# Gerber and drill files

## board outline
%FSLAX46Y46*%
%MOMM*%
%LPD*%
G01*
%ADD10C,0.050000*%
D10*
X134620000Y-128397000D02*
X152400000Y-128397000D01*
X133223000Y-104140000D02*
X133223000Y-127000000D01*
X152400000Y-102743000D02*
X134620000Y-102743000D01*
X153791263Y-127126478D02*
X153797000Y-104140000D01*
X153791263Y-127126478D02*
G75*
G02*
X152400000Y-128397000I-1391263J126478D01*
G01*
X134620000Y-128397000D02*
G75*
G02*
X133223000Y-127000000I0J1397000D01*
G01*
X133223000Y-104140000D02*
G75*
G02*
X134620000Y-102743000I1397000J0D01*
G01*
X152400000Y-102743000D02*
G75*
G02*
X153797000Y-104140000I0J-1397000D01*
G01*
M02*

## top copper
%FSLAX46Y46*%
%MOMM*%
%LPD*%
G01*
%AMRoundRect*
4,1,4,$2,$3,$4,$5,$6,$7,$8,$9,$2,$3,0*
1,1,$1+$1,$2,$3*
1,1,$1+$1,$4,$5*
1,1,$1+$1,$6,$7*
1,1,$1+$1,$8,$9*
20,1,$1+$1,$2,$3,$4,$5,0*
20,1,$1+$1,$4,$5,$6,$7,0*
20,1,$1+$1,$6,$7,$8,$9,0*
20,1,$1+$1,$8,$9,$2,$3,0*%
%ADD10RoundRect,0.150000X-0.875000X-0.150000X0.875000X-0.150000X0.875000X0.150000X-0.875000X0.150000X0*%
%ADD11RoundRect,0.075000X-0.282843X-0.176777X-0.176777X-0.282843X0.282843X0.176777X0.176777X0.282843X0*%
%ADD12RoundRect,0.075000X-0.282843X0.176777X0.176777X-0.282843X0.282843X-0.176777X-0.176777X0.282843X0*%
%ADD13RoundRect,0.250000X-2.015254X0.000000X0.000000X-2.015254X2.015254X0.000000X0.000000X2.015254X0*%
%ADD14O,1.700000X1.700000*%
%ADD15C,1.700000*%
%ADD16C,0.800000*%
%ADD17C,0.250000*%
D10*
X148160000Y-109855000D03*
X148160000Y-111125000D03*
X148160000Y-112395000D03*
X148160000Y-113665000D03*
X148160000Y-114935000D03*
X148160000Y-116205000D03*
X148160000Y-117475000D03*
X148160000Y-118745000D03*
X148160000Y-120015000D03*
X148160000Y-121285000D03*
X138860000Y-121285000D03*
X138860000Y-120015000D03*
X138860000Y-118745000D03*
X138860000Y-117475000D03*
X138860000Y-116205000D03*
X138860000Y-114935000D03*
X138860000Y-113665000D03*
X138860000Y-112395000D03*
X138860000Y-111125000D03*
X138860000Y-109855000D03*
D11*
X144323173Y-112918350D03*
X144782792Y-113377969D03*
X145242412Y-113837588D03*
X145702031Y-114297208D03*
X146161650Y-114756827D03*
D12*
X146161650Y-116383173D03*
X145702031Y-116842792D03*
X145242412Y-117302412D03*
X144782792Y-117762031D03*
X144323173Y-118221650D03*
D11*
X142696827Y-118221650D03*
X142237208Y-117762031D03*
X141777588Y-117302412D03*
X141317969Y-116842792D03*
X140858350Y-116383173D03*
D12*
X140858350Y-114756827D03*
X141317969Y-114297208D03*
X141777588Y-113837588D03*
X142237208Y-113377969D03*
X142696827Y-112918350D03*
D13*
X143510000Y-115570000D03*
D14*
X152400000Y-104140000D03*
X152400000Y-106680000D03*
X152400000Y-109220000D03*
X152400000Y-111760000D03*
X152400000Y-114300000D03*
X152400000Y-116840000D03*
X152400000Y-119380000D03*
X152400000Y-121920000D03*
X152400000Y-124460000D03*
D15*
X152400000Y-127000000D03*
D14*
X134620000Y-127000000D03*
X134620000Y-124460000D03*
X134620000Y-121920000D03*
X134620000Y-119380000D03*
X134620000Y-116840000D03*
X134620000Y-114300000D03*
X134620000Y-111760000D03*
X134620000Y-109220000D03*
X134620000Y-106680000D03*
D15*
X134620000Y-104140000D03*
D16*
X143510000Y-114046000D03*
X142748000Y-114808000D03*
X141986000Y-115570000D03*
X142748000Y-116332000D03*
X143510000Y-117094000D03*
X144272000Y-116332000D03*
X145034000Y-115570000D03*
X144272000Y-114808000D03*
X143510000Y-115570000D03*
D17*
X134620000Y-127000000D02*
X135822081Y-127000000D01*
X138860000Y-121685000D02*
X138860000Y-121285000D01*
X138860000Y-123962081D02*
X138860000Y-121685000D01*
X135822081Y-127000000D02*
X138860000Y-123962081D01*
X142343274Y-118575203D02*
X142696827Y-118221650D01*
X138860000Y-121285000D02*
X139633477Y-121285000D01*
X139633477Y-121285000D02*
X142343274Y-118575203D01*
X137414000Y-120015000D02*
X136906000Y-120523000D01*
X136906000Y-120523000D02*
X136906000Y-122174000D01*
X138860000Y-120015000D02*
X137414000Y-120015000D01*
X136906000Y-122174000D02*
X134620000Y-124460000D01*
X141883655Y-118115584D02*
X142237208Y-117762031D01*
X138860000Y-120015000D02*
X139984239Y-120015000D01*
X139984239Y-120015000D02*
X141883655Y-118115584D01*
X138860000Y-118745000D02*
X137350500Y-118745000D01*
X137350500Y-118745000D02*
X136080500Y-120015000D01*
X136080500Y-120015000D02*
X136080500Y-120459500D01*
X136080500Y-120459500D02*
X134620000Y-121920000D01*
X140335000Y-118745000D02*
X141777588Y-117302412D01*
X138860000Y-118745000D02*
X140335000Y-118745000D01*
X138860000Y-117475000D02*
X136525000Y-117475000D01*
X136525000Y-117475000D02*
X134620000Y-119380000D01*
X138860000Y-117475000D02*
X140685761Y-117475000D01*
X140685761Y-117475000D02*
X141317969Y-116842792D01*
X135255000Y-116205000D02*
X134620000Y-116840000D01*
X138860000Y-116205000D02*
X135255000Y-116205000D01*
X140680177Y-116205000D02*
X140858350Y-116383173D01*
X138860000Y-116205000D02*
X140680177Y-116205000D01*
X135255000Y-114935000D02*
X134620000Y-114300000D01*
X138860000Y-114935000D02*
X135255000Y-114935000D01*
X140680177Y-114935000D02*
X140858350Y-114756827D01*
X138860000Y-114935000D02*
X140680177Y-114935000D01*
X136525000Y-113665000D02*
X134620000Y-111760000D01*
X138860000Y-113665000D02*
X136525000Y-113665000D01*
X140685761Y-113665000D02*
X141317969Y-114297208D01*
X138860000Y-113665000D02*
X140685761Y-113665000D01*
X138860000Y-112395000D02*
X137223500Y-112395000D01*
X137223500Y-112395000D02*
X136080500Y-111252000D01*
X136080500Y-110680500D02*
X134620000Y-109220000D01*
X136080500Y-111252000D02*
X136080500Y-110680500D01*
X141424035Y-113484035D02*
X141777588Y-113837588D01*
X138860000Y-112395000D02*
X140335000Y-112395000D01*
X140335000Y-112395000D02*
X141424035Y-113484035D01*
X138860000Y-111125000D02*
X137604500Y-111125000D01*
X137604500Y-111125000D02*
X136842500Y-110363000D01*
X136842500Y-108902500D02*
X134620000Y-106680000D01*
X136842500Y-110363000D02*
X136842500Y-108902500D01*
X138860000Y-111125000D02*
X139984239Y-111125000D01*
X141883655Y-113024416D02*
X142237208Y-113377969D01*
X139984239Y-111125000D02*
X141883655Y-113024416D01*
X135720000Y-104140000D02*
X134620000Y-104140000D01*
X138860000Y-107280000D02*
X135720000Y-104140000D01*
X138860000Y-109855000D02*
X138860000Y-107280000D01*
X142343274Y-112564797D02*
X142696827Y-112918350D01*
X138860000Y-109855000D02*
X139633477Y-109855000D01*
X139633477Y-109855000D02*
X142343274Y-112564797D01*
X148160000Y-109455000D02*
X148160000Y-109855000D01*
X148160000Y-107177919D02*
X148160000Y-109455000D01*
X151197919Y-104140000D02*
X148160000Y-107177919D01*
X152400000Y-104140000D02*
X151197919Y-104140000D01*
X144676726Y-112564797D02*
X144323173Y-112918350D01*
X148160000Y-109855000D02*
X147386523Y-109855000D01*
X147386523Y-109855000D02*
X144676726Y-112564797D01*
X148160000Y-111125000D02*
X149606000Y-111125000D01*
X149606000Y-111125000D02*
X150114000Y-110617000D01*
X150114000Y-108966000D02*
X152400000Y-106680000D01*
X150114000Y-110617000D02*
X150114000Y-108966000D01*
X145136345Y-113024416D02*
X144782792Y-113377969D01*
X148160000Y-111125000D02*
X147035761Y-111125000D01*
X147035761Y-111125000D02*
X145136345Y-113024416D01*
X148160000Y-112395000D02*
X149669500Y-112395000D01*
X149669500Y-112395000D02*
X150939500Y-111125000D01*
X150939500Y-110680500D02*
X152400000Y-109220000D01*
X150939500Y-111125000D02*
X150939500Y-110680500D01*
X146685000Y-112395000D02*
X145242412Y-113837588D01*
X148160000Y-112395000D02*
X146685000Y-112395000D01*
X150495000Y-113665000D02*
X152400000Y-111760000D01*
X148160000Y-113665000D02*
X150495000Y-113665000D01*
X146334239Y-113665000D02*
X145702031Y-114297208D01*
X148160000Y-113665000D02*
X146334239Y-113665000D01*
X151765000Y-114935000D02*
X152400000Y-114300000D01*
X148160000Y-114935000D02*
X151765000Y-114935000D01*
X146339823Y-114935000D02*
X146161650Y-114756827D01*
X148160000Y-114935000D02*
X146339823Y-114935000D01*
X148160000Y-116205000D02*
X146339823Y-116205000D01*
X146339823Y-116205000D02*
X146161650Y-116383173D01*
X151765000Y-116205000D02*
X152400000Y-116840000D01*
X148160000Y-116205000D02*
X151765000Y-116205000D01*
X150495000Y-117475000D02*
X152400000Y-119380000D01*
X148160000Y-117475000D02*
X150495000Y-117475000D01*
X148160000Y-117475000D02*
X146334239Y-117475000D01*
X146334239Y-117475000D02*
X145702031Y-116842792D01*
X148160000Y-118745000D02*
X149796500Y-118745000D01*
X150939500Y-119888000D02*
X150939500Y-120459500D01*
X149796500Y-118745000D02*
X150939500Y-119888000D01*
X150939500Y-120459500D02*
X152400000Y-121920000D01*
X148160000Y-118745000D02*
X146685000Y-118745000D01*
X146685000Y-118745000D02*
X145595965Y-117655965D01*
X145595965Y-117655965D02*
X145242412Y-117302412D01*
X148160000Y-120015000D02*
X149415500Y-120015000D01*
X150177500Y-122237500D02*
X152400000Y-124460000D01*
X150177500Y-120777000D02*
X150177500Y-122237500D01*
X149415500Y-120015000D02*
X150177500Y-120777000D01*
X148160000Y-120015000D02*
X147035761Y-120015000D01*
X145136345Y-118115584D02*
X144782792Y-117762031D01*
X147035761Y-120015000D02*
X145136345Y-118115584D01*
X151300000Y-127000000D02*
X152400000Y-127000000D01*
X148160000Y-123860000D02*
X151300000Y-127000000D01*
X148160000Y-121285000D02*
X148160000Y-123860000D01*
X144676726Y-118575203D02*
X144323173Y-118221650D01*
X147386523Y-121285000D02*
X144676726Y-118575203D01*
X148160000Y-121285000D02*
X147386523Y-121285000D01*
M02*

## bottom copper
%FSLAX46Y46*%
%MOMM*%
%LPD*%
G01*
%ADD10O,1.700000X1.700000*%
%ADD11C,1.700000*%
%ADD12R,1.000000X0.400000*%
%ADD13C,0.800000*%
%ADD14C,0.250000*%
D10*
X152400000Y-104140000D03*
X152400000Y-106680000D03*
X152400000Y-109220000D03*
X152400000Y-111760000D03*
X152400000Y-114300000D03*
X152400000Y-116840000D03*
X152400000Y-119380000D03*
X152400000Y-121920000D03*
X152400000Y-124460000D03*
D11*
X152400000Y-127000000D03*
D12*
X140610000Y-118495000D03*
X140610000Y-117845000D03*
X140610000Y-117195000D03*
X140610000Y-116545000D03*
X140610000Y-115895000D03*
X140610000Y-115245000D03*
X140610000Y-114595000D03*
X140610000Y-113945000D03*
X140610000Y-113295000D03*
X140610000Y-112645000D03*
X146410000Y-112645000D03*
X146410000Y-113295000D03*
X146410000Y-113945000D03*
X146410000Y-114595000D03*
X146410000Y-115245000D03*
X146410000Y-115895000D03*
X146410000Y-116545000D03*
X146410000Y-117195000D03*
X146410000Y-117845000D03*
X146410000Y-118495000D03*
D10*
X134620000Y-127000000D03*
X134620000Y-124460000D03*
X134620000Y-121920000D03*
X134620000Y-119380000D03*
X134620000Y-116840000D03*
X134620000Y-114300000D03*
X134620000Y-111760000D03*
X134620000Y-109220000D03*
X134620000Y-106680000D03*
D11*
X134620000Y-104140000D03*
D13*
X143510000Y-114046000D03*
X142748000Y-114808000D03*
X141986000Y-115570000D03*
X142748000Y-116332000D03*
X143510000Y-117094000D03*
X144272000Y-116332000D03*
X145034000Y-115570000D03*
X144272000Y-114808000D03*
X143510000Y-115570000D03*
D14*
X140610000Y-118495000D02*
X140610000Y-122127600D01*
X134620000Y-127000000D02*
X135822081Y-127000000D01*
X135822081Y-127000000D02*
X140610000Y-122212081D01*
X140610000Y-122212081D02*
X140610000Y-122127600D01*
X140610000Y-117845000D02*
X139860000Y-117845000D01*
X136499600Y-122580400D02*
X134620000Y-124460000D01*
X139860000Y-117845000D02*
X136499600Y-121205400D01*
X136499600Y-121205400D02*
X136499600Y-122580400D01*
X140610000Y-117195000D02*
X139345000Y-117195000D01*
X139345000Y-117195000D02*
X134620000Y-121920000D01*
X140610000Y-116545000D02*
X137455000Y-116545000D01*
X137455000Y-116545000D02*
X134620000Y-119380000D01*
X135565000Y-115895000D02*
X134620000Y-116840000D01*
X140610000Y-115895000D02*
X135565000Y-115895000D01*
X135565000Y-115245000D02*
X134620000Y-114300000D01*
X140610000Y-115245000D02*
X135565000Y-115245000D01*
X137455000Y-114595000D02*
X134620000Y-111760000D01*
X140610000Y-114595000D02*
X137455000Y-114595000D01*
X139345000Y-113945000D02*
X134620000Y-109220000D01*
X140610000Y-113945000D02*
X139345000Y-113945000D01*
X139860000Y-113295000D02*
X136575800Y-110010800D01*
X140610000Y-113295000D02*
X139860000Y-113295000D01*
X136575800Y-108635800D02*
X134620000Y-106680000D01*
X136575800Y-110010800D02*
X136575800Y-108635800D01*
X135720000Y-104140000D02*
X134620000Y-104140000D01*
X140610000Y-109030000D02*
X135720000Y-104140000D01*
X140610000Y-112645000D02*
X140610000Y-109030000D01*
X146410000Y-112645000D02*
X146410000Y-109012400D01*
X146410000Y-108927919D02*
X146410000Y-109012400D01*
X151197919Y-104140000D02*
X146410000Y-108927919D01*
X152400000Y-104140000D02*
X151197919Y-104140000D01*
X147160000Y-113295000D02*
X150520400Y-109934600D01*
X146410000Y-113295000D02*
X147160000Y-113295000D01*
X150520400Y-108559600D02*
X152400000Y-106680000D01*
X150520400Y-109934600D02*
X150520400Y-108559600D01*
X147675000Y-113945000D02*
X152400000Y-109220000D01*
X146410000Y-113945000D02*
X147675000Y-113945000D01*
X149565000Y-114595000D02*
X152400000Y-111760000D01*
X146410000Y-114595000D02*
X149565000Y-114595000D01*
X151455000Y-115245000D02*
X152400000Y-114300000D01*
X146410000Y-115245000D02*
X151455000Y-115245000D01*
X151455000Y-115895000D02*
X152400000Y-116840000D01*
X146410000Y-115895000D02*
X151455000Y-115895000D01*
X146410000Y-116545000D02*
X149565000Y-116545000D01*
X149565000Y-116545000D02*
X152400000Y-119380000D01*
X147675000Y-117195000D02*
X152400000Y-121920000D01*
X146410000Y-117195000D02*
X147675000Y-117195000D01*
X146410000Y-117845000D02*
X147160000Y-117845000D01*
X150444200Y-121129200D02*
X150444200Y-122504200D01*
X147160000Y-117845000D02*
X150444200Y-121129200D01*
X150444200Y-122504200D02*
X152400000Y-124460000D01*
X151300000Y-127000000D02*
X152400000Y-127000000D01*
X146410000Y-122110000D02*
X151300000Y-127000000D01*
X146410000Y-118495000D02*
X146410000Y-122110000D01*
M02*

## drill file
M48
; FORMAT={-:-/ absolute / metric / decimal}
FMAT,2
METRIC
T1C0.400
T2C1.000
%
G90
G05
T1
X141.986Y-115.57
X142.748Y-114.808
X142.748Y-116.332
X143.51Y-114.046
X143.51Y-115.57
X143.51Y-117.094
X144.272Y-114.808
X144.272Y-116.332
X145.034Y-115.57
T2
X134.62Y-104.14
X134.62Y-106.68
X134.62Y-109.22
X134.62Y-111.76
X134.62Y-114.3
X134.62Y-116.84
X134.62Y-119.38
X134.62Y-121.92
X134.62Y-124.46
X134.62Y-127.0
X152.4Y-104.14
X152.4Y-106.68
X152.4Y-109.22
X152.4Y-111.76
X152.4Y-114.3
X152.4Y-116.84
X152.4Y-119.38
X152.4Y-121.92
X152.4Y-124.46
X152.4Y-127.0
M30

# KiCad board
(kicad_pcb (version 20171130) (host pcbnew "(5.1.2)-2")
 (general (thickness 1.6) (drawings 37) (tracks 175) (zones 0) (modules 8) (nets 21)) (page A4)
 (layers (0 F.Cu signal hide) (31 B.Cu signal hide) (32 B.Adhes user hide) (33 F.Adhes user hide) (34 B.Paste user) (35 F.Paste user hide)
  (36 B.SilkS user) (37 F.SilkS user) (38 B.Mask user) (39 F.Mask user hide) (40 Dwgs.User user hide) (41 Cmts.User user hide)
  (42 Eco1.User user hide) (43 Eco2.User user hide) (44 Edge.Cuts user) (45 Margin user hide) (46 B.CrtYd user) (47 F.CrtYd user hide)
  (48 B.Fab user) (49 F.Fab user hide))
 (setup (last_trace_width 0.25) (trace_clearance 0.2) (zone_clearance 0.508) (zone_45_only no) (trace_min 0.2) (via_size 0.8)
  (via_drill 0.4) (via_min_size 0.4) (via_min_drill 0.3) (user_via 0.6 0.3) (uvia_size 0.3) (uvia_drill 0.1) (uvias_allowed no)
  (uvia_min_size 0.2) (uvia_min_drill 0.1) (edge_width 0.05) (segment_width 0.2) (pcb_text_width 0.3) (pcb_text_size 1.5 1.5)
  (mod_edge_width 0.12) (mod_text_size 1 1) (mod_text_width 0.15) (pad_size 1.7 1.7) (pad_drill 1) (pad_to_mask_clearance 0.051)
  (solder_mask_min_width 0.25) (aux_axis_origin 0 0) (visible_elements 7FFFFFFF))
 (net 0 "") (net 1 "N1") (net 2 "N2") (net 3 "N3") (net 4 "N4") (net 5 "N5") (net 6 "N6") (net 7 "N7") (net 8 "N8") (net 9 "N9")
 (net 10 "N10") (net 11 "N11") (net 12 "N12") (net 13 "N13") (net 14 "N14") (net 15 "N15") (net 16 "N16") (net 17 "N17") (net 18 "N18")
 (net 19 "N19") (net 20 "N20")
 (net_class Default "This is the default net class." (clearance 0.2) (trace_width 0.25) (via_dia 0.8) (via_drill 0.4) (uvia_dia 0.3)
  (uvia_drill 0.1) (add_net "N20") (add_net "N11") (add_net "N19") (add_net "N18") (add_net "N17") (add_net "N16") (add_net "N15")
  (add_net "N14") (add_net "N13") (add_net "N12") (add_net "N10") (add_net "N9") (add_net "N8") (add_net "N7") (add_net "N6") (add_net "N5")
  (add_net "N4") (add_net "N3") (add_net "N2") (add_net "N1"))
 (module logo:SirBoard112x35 (layer B.Cu) (at 143.51 108.331)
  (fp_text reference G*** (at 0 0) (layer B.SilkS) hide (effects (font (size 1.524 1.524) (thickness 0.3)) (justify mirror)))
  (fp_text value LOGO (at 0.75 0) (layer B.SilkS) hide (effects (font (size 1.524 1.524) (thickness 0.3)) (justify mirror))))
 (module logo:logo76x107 (layer B.Cu) (at 143.51 123.952)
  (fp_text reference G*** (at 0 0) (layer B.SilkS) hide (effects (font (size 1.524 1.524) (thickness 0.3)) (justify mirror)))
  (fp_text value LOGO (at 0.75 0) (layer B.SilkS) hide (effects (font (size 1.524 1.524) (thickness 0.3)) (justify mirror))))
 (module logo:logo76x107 (layer F.Cu) (at 143.51 106.172 90)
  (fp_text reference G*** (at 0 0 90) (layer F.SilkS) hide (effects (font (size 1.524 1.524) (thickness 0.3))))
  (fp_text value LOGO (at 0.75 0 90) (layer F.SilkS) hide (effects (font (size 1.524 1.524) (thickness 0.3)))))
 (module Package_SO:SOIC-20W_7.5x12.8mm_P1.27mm (layer F.Cu) (at 143.51 115.57)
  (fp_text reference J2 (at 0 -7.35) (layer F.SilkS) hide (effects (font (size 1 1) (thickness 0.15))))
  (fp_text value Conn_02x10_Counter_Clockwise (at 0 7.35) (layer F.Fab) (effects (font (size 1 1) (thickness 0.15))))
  (pad 20 smd roundrect (at 4.65 -5.715) (size 2.05 0.6) (layers F.Cu F.Paste F.Mask) (roundrect_rratio 0.25) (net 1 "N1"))
  (pad 19 smd roundrect (at 4.65 -4.445) (size 2.05 0.6) (layers F.Cu F.Paste F.Mask) (roundrect_rratio 0.25) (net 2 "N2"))
  (pad 18 smd roundrect (at 4.65 -3.175) (size 2.05 0.6) (layers F.Cu F.Paste F.Mask) (roundrect_rratio 0.25) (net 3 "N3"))
  (pad 17 smd roundrect (at 4.65 -1.905) (size 2.05 0.6) (layers F.Cu F.Paste F.Mask) (roundrect_rratio 0.25) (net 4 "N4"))
  (pad 16 smd roundrect (at 4.65 -0.635) (size 2.05 0.6) (layers F.Cu F.Paste F.Mask) (roundrect_rratio 0.25) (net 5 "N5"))
  (pad 15 smd roundrect (at 4.65 0.635) (size 2.05 0.6) (layers F.Cu F.Paste F.Mask) (roundrect_rratio 0.25) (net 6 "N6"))
  (pad 14 smd roundrect (at 4.65 1.905) (size 2.05 0.6) (layers F.Cu F.Paste F.Mask) (roundrect_rratio 0.25) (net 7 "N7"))
  (pad 13 smd roundrect (at 4.65 3.175) (size 2.05 0.6) (layers F.Cu F.Paste F.Mask) (roundrect_rratio 0.25) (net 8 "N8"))
  (pad 12 smd roundrect (at 4.65 4.445) (size 2.05 0.6) (layers F.Cu F.Paste F.Mask) (roundrect_rratio 0.25) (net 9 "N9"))
  (pad 11 smd roundrect (at 4.65 5.715) (size 2.05 0.6) (layers F.Cu F.Paste F.Mask) (roundrect_rratio 0.25) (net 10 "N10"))
  (pad 10 smd roundrect (at -4.65 5.715) (size 2.05 0.6) (layers F.Cu F.Paste F.Mask) (roundrect_rratio 0.25) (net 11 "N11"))
  (pad 9 smd roundrect (at -4.65 4.445) (size 2.05 0.6) (layers F.Cu F.Paste F.Mask) (roundrect_rratio 0.25) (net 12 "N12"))
  (pad 8 smd roundrect (at -4.65 3.175) (size 2.05 0.6) (layers F.Cu F.Paste F.Mask) (roundrect_rratio 0.25) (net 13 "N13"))
  (pad 7 smd roundrect (at -4.65 1.905) (size 2.05 0.6) (layers F.Cu F.Paste F.Mask) (roundrect_rratio 0.25) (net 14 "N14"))
  (pad 6 smd roundrect (at -4.65 0.635) (size 2.05 0.6) (layers F.Cu F.Paste F.Mask) (roundrect_rratio 0.25) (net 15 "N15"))
  (pad 5 smd roundrect (at -4.65 -0.635) (size 2.05 0.6) (layers F.Cu F.Paste F.Mask) (roundrect_rratio 0.25) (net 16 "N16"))
  (pad 4 smd roundrect (at -4.65 -1.905) (size 2.05 0.6) (layers F.Cu F.Paste F.Mask) (roundrect_rratio 0.25) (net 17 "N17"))
  (pad 3 smd roundrect (at -4.65 -3.175) (size 2.05 0.6) (layers F.Cu F.Paste F.Mask) (roundrect_rratio 0.25) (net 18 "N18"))
  (pad 2 smd roundrect (at -4.65 -4.445) (size 2.05 0.6) (layers F.Cu F.Paste F.Mask) (roundrect_rratio 0.25) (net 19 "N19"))
  (pad 1 smd roundrect (at -4.65 -5.715) (size 2.05 0.6) (layers F.Cu F.Paste F.Mask) (roundrect_rratio 0.25) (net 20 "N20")))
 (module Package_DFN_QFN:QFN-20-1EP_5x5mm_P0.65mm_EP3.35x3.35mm (layer F.Cu) (at 143.51 115.57 315)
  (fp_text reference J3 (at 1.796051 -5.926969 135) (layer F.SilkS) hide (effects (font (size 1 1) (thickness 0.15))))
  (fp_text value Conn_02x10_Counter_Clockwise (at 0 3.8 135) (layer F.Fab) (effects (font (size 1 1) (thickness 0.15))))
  (pad 20 smd roundrect (at -1.3 -2.45 315) (size 0.3 0.8) (layers F.Cu F.Paste F.Mask) (roundrect_rratio 0.25) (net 1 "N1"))
  (pad 19 smd roundrect (at -0.65 -2.45 315) (size 0.3 0.8) (layers F.Cu F.Paste F.Mask) (roundrect_rratio 0.25) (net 2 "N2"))
  (pad 18 smd roundrect (at 0 -2.45 315) (size 0.3 0.8) (layers F.Cu F.Paste F.Mask) (roundrect_rratio 0.25) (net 3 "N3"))
  (pad 17 smd roundrect (at 0.65 -2.45 315) (size 0.3 0.8) (layers F.Cu F.Paste F.Mask) (roundrect_rratio 0.25) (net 4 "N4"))
  (pad 16 smd roundrect (at 1.3 -2.45 315) (size 0.3 0.8) (layers F.Cu F.Paste F.Mask) (roundrect_rratio 0.25) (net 5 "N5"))
  (pad 15 smd roundrect (at 2.45 -1.3 315) (size 0.8 0.3) (layers F.Cu F.Paste F.Mask) (roundrect_rratio 0.25) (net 6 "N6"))
  (pad 14 smd roundrect (at 2.45 -0.65 315) (size 0.8 0.3) (layers F.Cu F.Paste F.Mask) (roundrect_rratio 0.25) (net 7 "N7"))
  (pad 13 smd roundrect (at 2.45 0 315) (size 0.8 0.3) (layers F.Cu F.Paste F.Mask) (roundrect_rratio 0.25) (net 8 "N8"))
  (pad 12 smd roundrect (at 2.45 0.65 315) (size 0.8 0.3) (layers F.Cu F.Paste F.Mask) (roundrect_rratio 0.25) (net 9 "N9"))
  (pad 11 smd roundrect (at 2.45 1.3 315) (size 0.8 0.3) (layers F.Cu F.Paste F.Mask) (roundrect_rratio 0.25) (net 10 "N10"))
  (pad 10 smd roundrect (at 1.3 2.45 315) (size 0.3 0.8) (layers F.Cu F.Paste F.Mask) (roundrect_rratio 0.25) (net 11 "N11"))
  (pad 9 smd roundrect (at 0.65 2.45 315) (size 0.3 0.8) (layers F.Cu F.Paste F.Mask) (roundrect_rratio 0.25) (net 12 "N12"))
  (pad 8 smd roundrect (at 0 2.45 315) (size 0.3 0.8) (layers F.Cu F.Paste F.Mask) (roundrect_rratio 0.25) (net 13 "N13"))
  (pad 7 smd roundrect (at -0.65 2.45 315) (size 0.3 0.8) (layers F.Cu F.Paste F.Mask) (roundrect_rratio 0.25) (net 14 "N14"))
  (pad 6 smd roundrect (at -1.3 2.45 315) (size 0.3 0.8) (layers F.Cu F.Paste F.Mask) (roundrect_rratio 0.25) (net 15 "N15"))
  (pad 5 smd roundrect (at -2.45 1.3 315) (size 0.8 0.3) (layers F.Cu F.Paste F.Mask) (roundrect_rratio 0.25) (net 16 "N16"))
  (pad 4 smd roundrect (at -2.45 0.65 315) (size 0.8 0.3) (layers F.Cu F.Paste F.Mask) (roundrect_rratio 0.25) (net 17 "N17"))
  (pad 3 smd roundrect (at -2.45 0 315) (size 0.8 0.3) (layers F.Cu F.Paste F.Mask) (roundrect_rratio 0.25) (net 18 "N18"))
  (pad 2 smd roundrect (at -2.45 -0.65 315) (size 0.8 0.3) (layers F.Cu F.Paste F.Mask) (roundrect_rratio 0.25) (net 19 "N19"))
  (pad 1 smd roundrect (at -2.45 -1.3 315) (size 0.8 0.3) (layers F.Cu F.Paste F.Mask) (roundrect_rratio 0.25) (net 20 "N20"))
  (pad "" smd roundrect (at 0.84 0.84 315) (size 1.35 1.35) (layers F.Paste) (roundrect_rratio 0.185185))
  (pad "" smd roundrect (at 0.84 -0.84 315) (size 1.35 1.35) (layers F.Paste) (roundrect_rratio 0.185185))
  (pad "" smd roundrect (at -0.84 0.84 315) (size 1.35 1.35) (layers F.Paste) (roundrect_rratio 0.185185))
  (pad "" smd roundrect (at -0.84 -0.84 315) (size 1.35 1.35) (layers F.Paste) (roundrect_rratio 0.185185))
  (pad 21 smd roundrect (at 0 0 315) (size 3.35 3.35) (layers F.Cu F.Mask) (roundrect_rratio 0.074627)))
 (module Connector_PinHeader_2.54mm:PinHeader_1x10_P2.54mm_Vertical (layer F.Cu) (at 152.4 127 180)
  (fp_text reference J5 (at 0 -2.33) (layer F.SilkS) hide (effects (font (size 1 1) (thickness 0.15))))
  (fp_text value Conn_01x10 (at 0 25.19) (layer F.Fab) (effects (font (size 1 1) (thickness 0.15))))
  (pad 10 thru_hole oval (at 0 22.86 180) (size 1.7 1.7) (drill 1) (layers *.Cu *.Mask) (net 1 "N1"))
  (pad 9 thru_hole oval (at 0 20.32 180) (size 1.7 1.7) (drill 1) (layers *.Cu *.Mask) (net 2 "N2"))
  (pad 8 thru_hole oval (at 0 17.78 180) (size 1.7 1.7) (drill 1) (layers *.Cu *.Mask) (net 3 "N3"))
  (pad 7 thru_hole oval (at 0 15.24 180) (size 1.7 1.7) (drill 1) (layers *.Cu *.Mask) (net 4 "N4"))
  (pad 6 thru_hole oval (at 0 12.7 180) (size 1.7 1.7) (drill 1) (layers *.Cu *.Mask) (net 5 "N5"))
  (pad 5 thru_hole oval (at 0 10.16 180) (size 1.7 1.7) (drill 1) (layers *.Cu *.Mask) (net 6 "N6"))
  (pad 4 thru_hole oval (at 0 7.62 180) (size 1.7 1.7) (drill 1) (layers *.Cu *.Mask) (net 7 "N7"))
  (pad 3 thru_hole oval (at 0 5.08 180) (size 1.7 1.7) (drill 1) (layers *.Cu *.Mask) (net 8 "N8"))
  (pad 2 thru_hole oval (at 0 2.54 180) (size 1.7 1.7) (drill 1) (layers *.Cu *.Mask) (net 9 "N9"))
  (pad 1 thru_hole circle (at 0 0 180) (size 1.7 1.7) (drill 1) (layers *.Cu *.Mask) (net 10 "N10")))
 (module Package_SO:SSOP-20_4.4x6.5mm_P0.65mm (layer B.Cu) (at 143.51 115.57)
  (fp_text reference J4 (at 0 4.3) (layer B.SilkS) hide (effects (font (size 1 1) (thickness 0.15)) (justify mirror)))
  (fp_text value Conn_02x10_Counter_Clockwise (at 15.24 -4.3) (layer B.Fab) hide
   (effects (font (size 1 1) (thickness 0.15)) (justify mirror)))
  (pad 1 smd rect (at -2.9 2.925) (size 1 0.4) (layers B.Cu B.Paste B.Mask) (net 11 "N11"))
  (pad 2 smd rect (at -2.9 2.275) (size 1 0.4) (layers B.Cu B.Paste B.Mask) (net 12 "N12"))
  (pad 3 smd rect (at -2.9 1.625) (size 1 0.4) (layers B.Cu B.Paste B.Mask) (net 13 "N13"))
  (pad 4 smd rect (at -2.9 0.975) (size 1 0.4) (layers B.Cu B.Paste B.Mask) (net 14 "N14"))
  (pad 5 smd rect (at -2.9 0.325) (size 1 0.4) (layers B.Cu B.Paste B.Mask) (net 15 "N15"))
  (pad 6 smd rect (at -2.9 -0.325) (size 1 0.4) (layers B.Cu B.Paste B.Mask) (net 16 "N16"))
  (pad 7 smd rect (at -2.9 -0.975) (size 1 0.4) (layers B.Cu B.Paste B.Mask) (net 17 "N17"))
  (pad 8 smd rect (at -2.9 -1.625) (size 1 0.4) (layers B.Cu B.Paste B.Mask) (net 18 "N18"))
  (pad 9 smd rect (at -2.9 -2.275) (size 1 0.4) (layers B.Cu B.Paste B.Mask) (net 19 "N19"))
  (pad 10 smd rect (at -2.9 -2.925) (size 1 0.4) (layers B.Cu B.Paste B.Mask) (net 20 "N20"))
  (pad 11 smd rect (at 2.9 -2.925) (size 1 0.4) (layers B.Cu B.Paste B.Mask) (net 1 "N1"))
  (pad 12 smd rect (at 2.9 -2.275) (size 1 0.4) (layers B.Cu B.Paste B.Mask) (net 2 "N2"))
  (pad 13 smd rect (at 2.9 -1.625) (size 1 0.4) (layers B.Cu B.Paste B.Mask) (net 3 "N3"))
  (pad 14 smd rect (at 2.9 -0.975) (size 1 0.4) (layers B.Cu B.Paste B.Mask) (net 4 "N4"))
  (pad 15 smd rect (at 2.9 -0.325) (size 1 0.4) (layers B.Cu B.Paste B.Mask) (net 5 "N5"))
  (pad 16 smd rect (at 2.9 0.325) (size 1 0.4) (layers B.Cu B.Paste B.Mask) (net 6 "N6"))
  (pad 17 smd rect (at 2.9 0.975) (size 1 0.4) (layers B.Cu B.Paste B.Mask) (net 7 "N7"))
  (pad 18 smd rect (at 2.9 1.625) (size 1 0.4) (layers B.Cu B.Paste B.Mask) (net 8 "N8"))
  (pad 19 smd rect (at 2.9 2.275) (size 1 0.4) (layers B.Cu B.Paste B.Mask) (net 9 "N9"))
  (pad 20 smd rect (at 2.9 2.925) (size 1 0.4) (layers B.Cu B.Paste B.Mask) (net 10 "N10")))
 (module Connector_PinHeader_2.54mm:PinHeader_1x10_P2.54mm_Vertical (layer F.Cu) (at 134.62 104.14)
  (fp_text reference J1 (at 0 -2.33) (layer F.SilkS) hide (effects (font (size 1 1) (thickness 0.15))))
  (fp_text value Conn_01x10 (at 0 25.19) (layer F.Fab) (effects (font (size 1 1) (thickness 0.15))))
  (pad 10 thru_hole oval (at 0 22.86) (size 1.7 1.7) (drill 1) (layers *.Cu *.Mask) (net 11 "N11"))
  (pad 9 thru_hole oval (at 0 20.32) (size 1.7 1.7) (drill 1) (layers *.Cu *.Mask) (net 12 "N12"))
  (pad 8 thru_hole oval (at 0 17.78) (size 1.7 1.7) (drill 1) (layers *.Cu *.Mask) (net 13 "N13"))
  (pad 7 thru_hole oval (at 0 15.24) (size 1.7 1.7) (drill 1) (layers *.Cu *.Mask) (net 14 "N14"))
  (pad 6 thru_hole oval (at 0 12.7) (size 1.7 1.7) (drill 1) (layers *.Cu *.Mask) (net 15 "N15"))
  (pad 5 thru_hole oval (at 0 10.16) (size 1.7 1.7) (drill 1) (layers *.Cu *.Mask) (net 16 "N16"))
  (pad 4 thru_hole oval (at 0 7.62) (size 1.7 1.7) (drill 1) (layers *.Cu *.Mask) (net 17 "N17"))
  (pad 3 thru_hole oval (at 0 5.08) (size 1.7 1.7) (drill 1) (layers *.Cu *.Mask) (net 18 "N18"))
  (pad 2 thru_hole oval (at 0 2.54) (size 1.7 1.7) (drill 1) (layers *.Cu *.Mask) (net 19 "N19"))
  (pad 1 thru_hole circle (at 0 0) (size 1.7 1.7) (drill 1) (layers *.Cu *.Mask) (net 20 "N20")))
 (gr_line (start 134.62 128.397) (end 152.4 128.397) (layer Edge.Cuts) (width 0.05))
 (gr_line (start 133.223 104.14) (end 133.223 127) (layer Edge.Cuts) (width 0.05))
 (gr_line (start 152.4 102.743) (end 134.62 102.743) (layer Edge.Cuts) (width 0.05))
 (gr_line (start 153.791263 127.126478) (end 153.797 104.14) (layer Edge.Cuts) (width 0.05))
 (gr_arc (start 152.4 127) (end 152.4 128.397) (angle -84.80557109) (layer Edge.Cuts) (width 0.05))
 (gr_arc (start 134.62 127) (end 133.223 127) (angle -90) (layer Edge.Cuts) (width 0.05))
 (gr_arc (start 134.62 104.14) (end 134.62 102.743) (angle -90) (layer Edge.Cuts) (width 0.05))
 (gr_arc (start 152.4 104.14) (end 153.797 104.14) (angle -90) (layer Edge.Cuts) (width 0.05))
 (via (at 143.51 114.046) (size 0.8) (drill 0.4) (layers F.Cu B.Cu) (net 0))
 (via (at 142.748 114.808) (size 0.8) (drill 0.4) (layers F.Cu B.Cu) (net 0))
 (via (at 141.986 115.57) (size 0.8) (drill 0.4) (layers F.Cu B.Cu) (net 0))
 (via (at 142.748 116.332) (size 0.8) (drill 0.4) (layers F.Cu B.Cu) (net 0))
 (via (at 143.51 117.094) (size 0.8) (drill 0.4) (layers F.Cu B.Cu) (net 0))
 (via (at 144.272 116.332) (size 0.8) (drill 0.4) (layers F.Cu B.Cu) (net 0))
 (via (at 145.034 115.57) (size 0.8) (drill 0.4) (layers F.Cu B.Cu) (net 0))
 (via (at 144.272 114.808) (size 0.8) (drill 0.4) (layers F.Cu B.Cu) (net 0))
 (via (at 143.51 115.57) (size 0.8) (drill 0.4) (layers F.Cu B.Cu) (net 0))
 (segment (start 134.62 127) (end 135.822081 127) (width 0.25) (layer F.Cu) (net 11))
 (segment (start 138.86 121.685) (end 138.86 121.285) (width 0.25) (layer F.Cu) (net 11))
 (segment (start 138.86 123.962081) (end 138.86 121.685) (width 0.25) (layer F.Cu) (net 11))
 (segment (start 135.822081 127) (end 138.86 123.962081) (width 0.25) (layer F.Cu) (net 11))
 (segment (start 142.343274 118.575203) (end 142.696827 118.22165) (width 0.25) (layer F.Cu) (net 11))
 (segment (start 138.86 121.285) (end 139.633477 121.285) (width 0.25) (layer F.Cu) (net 11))
 (segment (start 139.633477 121.285) (end 142.343274 118.575203) (width 0.25) (layer F.Cu) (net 11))
 (segment (start 140.61 118.495) (end 140.61 122.1276) (width 0.25) (layer B.Cu) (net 11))
 (segment (start 134.62 127) (end 135.822081 127) (width 0.25) (layer B.Cu) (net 11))
 (segment (start 135.822081 127) (end 140.61 122.212081) (width 0.25) (layer B.Cu) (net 11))
 (segment (start 140.61 122.212081) (end 140.61 122.1276) (width 0.25) (layer B.Cu) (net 11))
 (segment (start 137.414 120.015) (end 136.906 120.523) (width 0.25) (layer F.Cu) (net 12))
 (segment (start 136.906 120.523) (end 136.906 122.174) (width 0.25) (layer F.Cu) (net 12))
 (segment (start 138.86 120.015) (end 137.414 120.015) (width 0.25) (layer F.Cu) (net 12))
 (segment (start 136.906 122.174) (end 134.62 124.46) (width 0.25) (layer F.Cu) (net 12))
 (segment (start 141.883655 118.115584) (end 142.237208 117.762031) (width 0.25) (layer F.Cu) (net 12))
 (segment (start 138.86 120.015) (end 139.984239 120.015) (width 0.25) (layer F.Cu) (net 12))
 (segment (start 139.984239 120.015) (end 141.883655 118.115584) (width 0.25) (layer F.Cu) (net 12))
 (segment (start 140.61 117.845) (end 139.86 117.845) (width 0.25) (layer B.Cu) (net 12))
 (segment (start 136.4996 122.5804) (end 134.62 124.46) (width 0.25) (layer B.Cu) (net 12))
 (segment (start 139.86 117.845) (end 136.4996 121.2054) (width 0.25) (layer B.Cu) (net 12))
 (segment (start 136.4996 121.2054) (end 136.4996 122.5804) (width 0.25) (layer B.Cu) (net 12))
 (segment (start 138.86 118.745) (end 137.3505 118.745) (width 0.25) (layer F.Cu) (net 13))
 (segment (start 137.3505 118.745) (end 136.0805 120.015) (width 0.25) (layer F.Cu) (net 13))
 (segment (start 136.0805 120.015) (end 136.0805 120.4595) (width 0.25) (layer F.Cu) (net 13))
 (segment (start 136.0805 120.4595) (end 134.62 121.92) (width 0.25) (layer F.Cu) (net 13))
 (segment (start 140.335 118.745) (end 141.777588 117.302412) (width 0.25) (layer F.Cu) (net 13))
 (segment (start 138.86 118.745) (end 140.335 118.745) (width 0.25) (layer F.Cu) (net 13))
 (segment (start 140.61 117.195) (end 139.345 117.195) (width 0.25) (layer B.Cu) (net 13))
 (segment (start 139.345 117.195) (end 134.62 121.92) (width 0.25) (layer B.Cu) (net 13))
 (segment (start 138.86 117.475) (end 136.525 117.475) (width 0.25) (layer F.Cu) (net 14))
 (segment (start 136.525 117.475) (end 134.62 119.38) (width 0.25) (layer F.Cu) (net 14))
 (segment (start 138.86 117.475) (end 140.685761 117.475) (width 0.25) (layer F.Cu) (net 14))
 (segment (start 140.685761 117.475) (end 141.317969 116.842792) (width 0.25) (layer F.Cu) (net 14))
 (segment (start 140.61 116.545) (end 137.455 116.545) (width 0.25) (layer B.Cu) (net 14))
 (segment (start 137.455 116.545) (end 134.62 119.38) (width 0.25) (layer B.Cu) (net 14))
 (segment (start 135.255 116.205) (end 134.62 116.84) (width 0.25) (layer F.Cu) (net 15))
 (segment (start 138.86 116.205) (end 135.255 116.205) (width 0.25) (layer F.Cu) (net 15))
 (segment (start 140.680177 116.205) (end 140.85835 116.383173) (width 0.25) (layer F.Cu) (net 15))
 (segment (start 138.86 116.205) (end 140.680177 116.205) (width 0.25) (layer F.Cu) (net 15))
 (segment (start 135.565 115.895) (end 134.62 116.84) (width 0.25) (layer B.Cu) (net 15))
 (segment (start 140.61 115.895) (end 135.565 115.895) (width 0.25) (layer B.Cu) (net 15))
 (segment (start 135.255 114.935) (end 134.62 114.3) (width 0.25) (layer F.Cu) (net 16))
 (segment (start 138.86 114.935) (end 135.255 114.935) (width 0.25) (layer F.Cu) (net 16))
 (segment (start 140.680177 114.935) (end 140.85835 114.756827) (width 0.25) (layer F.Cu) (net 16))
 (segment (start 138.86 114.935) (end 140.680177 114.935) (width 0.25) (layer F.Cu) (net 16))
 (segment (start 135.565 115.245) (end 134.62 114.3) (width 0.25) (layer B.Cu) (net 16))
 (segment (start 140.61 115.245) (end 135.565 115.245) (width 0.25) (layer B.Cu) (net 16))
 (segment (start 136.525 113.665) (end 134.62 111.76) (width 0.25) (layer F.Cu) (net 17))
 (segment (start 138.86 113.665) (end 136.525 113.665) (width 0.25) (layer F.Cu) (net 17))
 (segment (start 140.685761 113.665) (end 141.317969 114.297208) (width 0.25) (layer F.Cu) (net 17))
 (segment (start 138.86 113.665) (end 140.685761 113.665) (width 0.25) (layer F.Cu) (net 17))
 (segment (start 137.455 114.595) (end 134.62 111.76) (width 0.25) (layer B.Cu) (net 17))
 (segment (start 140.61 114.595) (end 137.455 114.595) (width 0.25) (layer B.Cu) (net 17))
 (segment (start 138.86 112.395) (end 137.2235 112.395) (width 0.25) (layer F.Cu) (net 18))
 (segment (start 137.2235 112.395) (end 136.0805 111.252) (width 0.25) (layer F.Cu) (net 18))
 (segment (start 136.0805 110.6805) (end 134.62 109.22) (width 0.25) (layer F.Cu) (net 18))
 (segment (start 136.0805 111.252) (end 136.0805 110.6805) (width 0.25) (layer F.Cu) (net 18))
 (segment (start 141.424035 113.484035) (end 141.777588 113.837588) (width 0.25) (layer F.Cu) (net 18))
 (segment (start 138.86 112.395) (end 140.335 112.395) (width 0.25) (layer F.Cu) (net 18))
 (segment (start 140.335 112.395) (end 141.424035 113.484035) (width 0.25) (layer F.Cu) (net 18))
 (segment (start 139.345 113.945) (end 134.62 109.22) (width 0.25) (layer B.Cu) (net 18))
 (segment (start 140.61 113.945) (end 139.345 113.945) (width 0.25) (layer B.Cu) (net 18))
 (segment (start 138.86 111.125) (end 137.6045 111.125) (width 0.25) (layer F.Cu) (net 19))
 (segment (start 137.6045 111.125) (end 136.8425 110.363) (width 0.25) (layer F.Cu) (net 19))
 (segment (start 136.8425 108.9025) (end 134.62 106.68) (width 0.25) (layer F.Cu) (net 19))
 (segment (start 136.8425 110.363) (end 136.8425 108.9025) (width 0.25) (layer F.Cu) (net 19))
 (segment (start 138.86 111.125) (end 139.984239 111.125) (width 0.25) (layer F.Cu) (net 19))
 (segment (start 141.883655 113.024416) (end 142.237208 113.377969) (width 0.25) (layer F.Cu) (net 19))
 (segment (start 139.984239 111.125) (end 141.883655 113.024416) (width 0.25) (layer F.Cu) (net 19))
 (segment (start 139.86 113.295) (end 136.5758 110.0108) (width 0.25) (layer B.Cu) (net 19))
 (segment (start 140.61 113.295) (end 139.86 113.295) (width 0.25) (layer B.Cu) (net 19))
 (segment (start 136.5758 108.6358) (end 134.62 106.68) (width 0.25) (layer B.Cu) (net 19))
 (segment (start 136.5758 110.0108) (end 136.5758 108.6358) (width 0.25) (layer B.Cu) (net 19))
 (segment (start 135.72 104.14) (end 134.62 104.14) (width 0.25) (layer F.Cu) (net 20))
 (segment (start 138.86 107.28) (end 135.72 104.14) (width 0.25) (layer F.Cu) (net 20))
 (segment (start 138.86 109.855) (end 138.86 107.28) (width 0.25) (layer F.Cu) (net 20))
 (segment (start 142.343274 112.564797) (end 142.696827 112.91835) (width 0.25) (layer F.Cu) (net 20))
 (segment (start 138.86 109.855) (end 139.633477 109.855) (width 0.25) (layer F.Cu) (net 20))
 (segment (start 139.633477 109.855) (end 142.343274 112.564797) (width 0.25) (layer F.Cu) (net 20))
 (segment (start 135.72 104.14) (end 134.62 104.14) (width 0.25) (layer B.Cu) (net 20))
 (segment (start 140.61 109.03) (end 135.72 104.14) (width 0.25) (layer B.Cu) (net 20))
 (segment (start 140.61 112.645) (end 140.61 109.03) (width 0.25) (layer B.Cu) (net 20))
 (segment (start 148.16 109.455) (end 148.16 109.855) (width 0.25) (layer F.Cu) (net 1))
 (segment (start 148.16 107.177919) (end 148.16 109.455) (width 0.25) (layer F.Cu) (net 1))
 (segment (start 151.197919 104.14) (end 148.16 107.177919) (width 0.25) (layer F.Cu) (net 1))
 (segment (start 152.4 104.14) (end 151.197919 104.14) (width 0.25) (layer F.Cu) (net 1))
 (segment (start 144.676726 112.564797) (end 144.323173 112.91835) (width 0.25) (layer F.Cu) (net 1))
 (segment (start 148.16 109.855) (end 147.386523 109.855) (width 0.25) (layer F.Cu) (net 1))
 (segment (start 147.386523 109.855) (end 144.676726 112.564797) (width 0.25) (layer F.Cu) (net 1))
 (segment (start 146.41 112.645) (end 146.41 109.0124) (width 0.25) (layer B.Cu) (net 1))
 (segment (start 146.41 108.927919) (end 146.41 109.0124) (width 0.25) (layer B.Cu) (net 1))
 (segment (start 151.197919 104.14) (end 146.41 108.927919) (width 0.25) (layer B.Cu) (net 1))
 (segment (start 152.4 104.14) (end 151.197919 104.14) (width 0.25) (layer B.Cu) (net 1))
 (segment (start 148.16 111.125) (end 149.606 111.125) (width 0.25) (layer F.Cu) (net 2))
 (segment (start 149.606 111.125) (end 150.114 110.617) (width 0.25) (layer F.Cu) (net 2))
 (segment (start 150.114 108.966) (end 152.4 106.68) (width 0.25) (layer F.Cu) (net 2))
 (segment (start 150.114 110.617) (end 150.114 108.966) (width 0.25) (layer F.Cu) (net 2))
 (segment (start 145.136345 113.024416) (end 144.782792 113.377969) (width 0.25) (layer F.Cu) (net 2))
 (segment (start 148.16 111.125) (end 147.035761 111.125) (width 0.25) (layer F.Cu) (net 2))
 (segment (start 147.035761 111.125) (end 145.136345 113.024416) (width 0.25) (layer F.Cu) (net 2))
 (segment (start 147.16 113.295) (end 150.5204 109.9346) (width 0.25) (layer B.Cu) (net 2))
 (segment (start 146.41 113.295) (end 147.16 113.295) (width 0.25) (layer B.Cu) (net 2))
 (segment (start 150.5204 108.5596) (end 152.4 106.68) (width 0.25) (layer B.Cu) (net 2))
 (segment (start 150.5204 109.9346) (end 150.5204 108.5596) (width 0.25) (layer B.Cu) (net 2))
 (segment (start 148.16 112.395) (end 149.6695 112.395) (width 0.25) (layer F.Cu) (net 3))
 (segment (start 149.6695 112.395) (end 150.9395 111.125) (width 0.25) (layer F.Cu) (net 3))
 (segment (start 150.9395 110.6805) (end 152.4 109.22) (width 0.25) (layer F.Cu) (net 3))
 (segment (start 150.9395 111.125) (end 150.9395 110.6805) (width 0.25) (layer F.Cu) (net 3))
 (segment (start 146.685 112.395) (end 145.242412 113.837588) (width 0.25) (layer F.Cu) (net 3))
 (segment (start 148.16 112.395) (end 146.685 112.395) (width 0.25) (layer F.Cu) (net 3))
 (segment (start 147.675 113.945) (end 152.4 109.22) (width 0.25) (layer B.Cu) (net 3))
 (segment (start 146.41 113.945) (end 147.675 113.945) (width 0.25) (layer B.Cu) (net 3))
 (segment (start 150.495 113.665) (end 152.4 111.76) (width 0.25) (layer F.Cu) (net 4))
 (segment (start 148.16 113.665) (end 150.495 113.665) (width 0.25) (layer F.Cu) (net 4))
 (segment (start 146.334239 113.665) (end 145.702031 114.297208) (width 0.25) (layer F.Cu) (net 4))
 (segment (start 148.16 113.665) (end 146.334239 113.665) (width 0.25) (layer F.Cu) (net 4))
 (segment (start 149.565 114.595) (end 152.4 111.76) (width 0.25) (layer B.Cu) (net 4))
 (segment (start 146.41 114.595) (end 149.565 114.595) (width 0.25) (layer B.Cu) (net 4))
 (segment (start 151.765 114.935) (end 152.4 114.3) (width 0.25) (layer F.Cu) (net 5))
 (segment (start 148.16 114.935) (end 151.765 114.935) (width 0.25) (layer F.Cu) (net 5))
 (segment (start 146.339823 114.935) (end 146.16165 114.756827) (width 0.25) (layer F.Cu) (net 5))
 (segment (start 148.16 114.935) (end 146.339823 114.935) (width 0.25) (layer F.Cu) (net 5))
 (segment (start 151.455 115.245) (end 152.4 114.3) (width 0.25) (layer B.Cu) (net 5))
 (segment (start 146.41 115.245) (end 151.455 115.245) (width 0.25) (layer B.Cu) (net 5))
 (segment (start 148.16 116.205) (end 146.339823 116.205) (width 0.25) (layer F.Cu) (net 6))
 (segment (start 146.339823 116.205) (end 146.16165 116.383173) (width 0.25) (layer F.Cu) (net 6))
 (segment (start 151.765 116.205) (end 152.4 116.84) (width 0.25) (layer F.Cu) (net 6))
 (segment (start 148.16 116.205) (end 151.765 116.205) (width 0.25) (layer F.Cu) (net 6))
 (segment (start 151.455 115.895) (end 152.4 116.84) (width 0.25) (layer B.Cu) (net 6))
 (segment (start 146.41 115.895) (end 151.455 115.895) (width 0.25) (layer B.Cu) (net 6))
 (segment (start 150.495 117.475) (end 152.4 119.38) (width 0.25) (layer F.Cu) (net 7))
 (segment (start 148.16 117.475) (end 150.495 117.475) (width 0.25) (layer F.Cu) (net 7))
 (segment (start 148.16 117.475) (end 146.334239 117.475) (width 0.25) (layer F.Cu) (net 7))
 (segment (start 146.334239 117.475) (end 145.702031 116.842792) (width 0.25) (layer F.Cu) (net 7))
 (segment (start 146.41 116.545) (end 149.565 116.545) (width 0.25) (layer B.Cu) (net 7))
 (segment (start 149.565 116.545) (end 152.4 119.38) (width 0.25) (layer B.Cu) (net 7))
 (segment (start 148.16 118.745) (end 149.7965 118.745) (width 0.25) (layer F.Cu) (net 8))
 (segment (start 150.9395 119.888) (end 150.9395 120.4595) (width 0.25) (layer F.Cu) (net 8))
 (segment (start 149.7965 118.745) (end 150.9395 119.888) (width 0.25) (layer F.Cu) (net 8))
 (segment (start 150.9395 120.4595) (end 152.4 121.92) (width 0.25) (layer F.Cu) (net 8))
 (segment (start 148.16 118.745) (end 146.685 118.745) (width 0.25) (layer F.Cu) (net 8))
 (segment (start 146.685 118.745) (end 145.595965 117.655965) (width 0.25) (layer F.Cu) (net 8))
 (segment (start 145.595965 117.655965) (end 145.242412 117.302412) (width 0.25) (layer F.Cu) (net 8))
 (segment (start 147.675 117.195) (end 152.4 121.92) (width 0.25) (layer B.Cu) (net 8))
 (segment (start 146.41 117.195) (end 147.675 117.195) (width 0.25) (layer B.Cu) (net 8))
 (segment (start 148.16 120.015) (end 149.4155 120.015) (width 0.25) (layer F.Cu) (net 9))
 (segment (start 150.1775 122.2375) (end 152.4 124.46) (width 0.25) (layer F.Cu) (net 9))
 (segment (start 150.1775 120.777) (end 150.1775 122.2375) (width 0.25) (layer F.Cu) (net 9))
 (segment (start 149.4155 120.015) (end 150.1775 120.777) (width 0.25) (layer F.Cu) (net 9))
 (segment (start 148.16 120.015) (end 147.035761 120.015) (width 0.25) (layer F.Cu) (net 9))
 (segment (start 145.136345 118.115584) (end 144.782792 117.762031) (width 0.25) (layer F.Cu) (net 9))
 (segment (start 147.035761 120.015) (end 145.136345 118.115584) (width 0.25) (layer F.Cu) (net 9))
 (segment (start 146.41 117.845) (end 147.16 117.845) (width 0.25) (layer B.Cu) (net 9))
 (segment (start 150.4442 121.1292) (end 150.4442 122.5042) (width 0.25) (layer B.Cu) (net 9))
 (segment (start 147.16 117.845) (end 150.4442 121.1292) (width 0.25) (layer B.Cu) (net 9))
 (segment (start 150.4442 122.5042) (end 152.4 124.46) (width 0.25) (layer B.Cu) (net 9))
 (segment (start 151.3 127) (end 152.4 127) (width 0.25) (layer F.Cu) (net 10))
 (segment (start 148.16 123.86) (end 151.3 127) (width 0.25) (layer F.Cu) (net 10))
 (segment (start 148.16 121.285) (end 148.16 123.86) (width 0.25) (layer F.Cu) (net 10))
 (segment (start 144.676726 118.575203) (end 144.323173 118.22165) (width 0.25) (layer F.Cu) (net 10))
 (segment (start 147.386523 121.285) (end 144.676726 118.575203) (width 0.25) (layer F.Cu) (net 10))
 (segment (start 148.16 121.285) (end 147.386523 121.285) (width 0.25) (layer F.Cu) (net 10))
 (segment (start 151.3 127) (end 152.4 127) (width 0.25) (layer B.Cu) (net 10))
 (segment (start 146.41 122.11) (end 151.3 127) (width 0.25) (layer B.Cu) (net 10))
 (segment (start 146.41 118.495) (end 146.41 122.11) (width 0.25) (layer B.Cu) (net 10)))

